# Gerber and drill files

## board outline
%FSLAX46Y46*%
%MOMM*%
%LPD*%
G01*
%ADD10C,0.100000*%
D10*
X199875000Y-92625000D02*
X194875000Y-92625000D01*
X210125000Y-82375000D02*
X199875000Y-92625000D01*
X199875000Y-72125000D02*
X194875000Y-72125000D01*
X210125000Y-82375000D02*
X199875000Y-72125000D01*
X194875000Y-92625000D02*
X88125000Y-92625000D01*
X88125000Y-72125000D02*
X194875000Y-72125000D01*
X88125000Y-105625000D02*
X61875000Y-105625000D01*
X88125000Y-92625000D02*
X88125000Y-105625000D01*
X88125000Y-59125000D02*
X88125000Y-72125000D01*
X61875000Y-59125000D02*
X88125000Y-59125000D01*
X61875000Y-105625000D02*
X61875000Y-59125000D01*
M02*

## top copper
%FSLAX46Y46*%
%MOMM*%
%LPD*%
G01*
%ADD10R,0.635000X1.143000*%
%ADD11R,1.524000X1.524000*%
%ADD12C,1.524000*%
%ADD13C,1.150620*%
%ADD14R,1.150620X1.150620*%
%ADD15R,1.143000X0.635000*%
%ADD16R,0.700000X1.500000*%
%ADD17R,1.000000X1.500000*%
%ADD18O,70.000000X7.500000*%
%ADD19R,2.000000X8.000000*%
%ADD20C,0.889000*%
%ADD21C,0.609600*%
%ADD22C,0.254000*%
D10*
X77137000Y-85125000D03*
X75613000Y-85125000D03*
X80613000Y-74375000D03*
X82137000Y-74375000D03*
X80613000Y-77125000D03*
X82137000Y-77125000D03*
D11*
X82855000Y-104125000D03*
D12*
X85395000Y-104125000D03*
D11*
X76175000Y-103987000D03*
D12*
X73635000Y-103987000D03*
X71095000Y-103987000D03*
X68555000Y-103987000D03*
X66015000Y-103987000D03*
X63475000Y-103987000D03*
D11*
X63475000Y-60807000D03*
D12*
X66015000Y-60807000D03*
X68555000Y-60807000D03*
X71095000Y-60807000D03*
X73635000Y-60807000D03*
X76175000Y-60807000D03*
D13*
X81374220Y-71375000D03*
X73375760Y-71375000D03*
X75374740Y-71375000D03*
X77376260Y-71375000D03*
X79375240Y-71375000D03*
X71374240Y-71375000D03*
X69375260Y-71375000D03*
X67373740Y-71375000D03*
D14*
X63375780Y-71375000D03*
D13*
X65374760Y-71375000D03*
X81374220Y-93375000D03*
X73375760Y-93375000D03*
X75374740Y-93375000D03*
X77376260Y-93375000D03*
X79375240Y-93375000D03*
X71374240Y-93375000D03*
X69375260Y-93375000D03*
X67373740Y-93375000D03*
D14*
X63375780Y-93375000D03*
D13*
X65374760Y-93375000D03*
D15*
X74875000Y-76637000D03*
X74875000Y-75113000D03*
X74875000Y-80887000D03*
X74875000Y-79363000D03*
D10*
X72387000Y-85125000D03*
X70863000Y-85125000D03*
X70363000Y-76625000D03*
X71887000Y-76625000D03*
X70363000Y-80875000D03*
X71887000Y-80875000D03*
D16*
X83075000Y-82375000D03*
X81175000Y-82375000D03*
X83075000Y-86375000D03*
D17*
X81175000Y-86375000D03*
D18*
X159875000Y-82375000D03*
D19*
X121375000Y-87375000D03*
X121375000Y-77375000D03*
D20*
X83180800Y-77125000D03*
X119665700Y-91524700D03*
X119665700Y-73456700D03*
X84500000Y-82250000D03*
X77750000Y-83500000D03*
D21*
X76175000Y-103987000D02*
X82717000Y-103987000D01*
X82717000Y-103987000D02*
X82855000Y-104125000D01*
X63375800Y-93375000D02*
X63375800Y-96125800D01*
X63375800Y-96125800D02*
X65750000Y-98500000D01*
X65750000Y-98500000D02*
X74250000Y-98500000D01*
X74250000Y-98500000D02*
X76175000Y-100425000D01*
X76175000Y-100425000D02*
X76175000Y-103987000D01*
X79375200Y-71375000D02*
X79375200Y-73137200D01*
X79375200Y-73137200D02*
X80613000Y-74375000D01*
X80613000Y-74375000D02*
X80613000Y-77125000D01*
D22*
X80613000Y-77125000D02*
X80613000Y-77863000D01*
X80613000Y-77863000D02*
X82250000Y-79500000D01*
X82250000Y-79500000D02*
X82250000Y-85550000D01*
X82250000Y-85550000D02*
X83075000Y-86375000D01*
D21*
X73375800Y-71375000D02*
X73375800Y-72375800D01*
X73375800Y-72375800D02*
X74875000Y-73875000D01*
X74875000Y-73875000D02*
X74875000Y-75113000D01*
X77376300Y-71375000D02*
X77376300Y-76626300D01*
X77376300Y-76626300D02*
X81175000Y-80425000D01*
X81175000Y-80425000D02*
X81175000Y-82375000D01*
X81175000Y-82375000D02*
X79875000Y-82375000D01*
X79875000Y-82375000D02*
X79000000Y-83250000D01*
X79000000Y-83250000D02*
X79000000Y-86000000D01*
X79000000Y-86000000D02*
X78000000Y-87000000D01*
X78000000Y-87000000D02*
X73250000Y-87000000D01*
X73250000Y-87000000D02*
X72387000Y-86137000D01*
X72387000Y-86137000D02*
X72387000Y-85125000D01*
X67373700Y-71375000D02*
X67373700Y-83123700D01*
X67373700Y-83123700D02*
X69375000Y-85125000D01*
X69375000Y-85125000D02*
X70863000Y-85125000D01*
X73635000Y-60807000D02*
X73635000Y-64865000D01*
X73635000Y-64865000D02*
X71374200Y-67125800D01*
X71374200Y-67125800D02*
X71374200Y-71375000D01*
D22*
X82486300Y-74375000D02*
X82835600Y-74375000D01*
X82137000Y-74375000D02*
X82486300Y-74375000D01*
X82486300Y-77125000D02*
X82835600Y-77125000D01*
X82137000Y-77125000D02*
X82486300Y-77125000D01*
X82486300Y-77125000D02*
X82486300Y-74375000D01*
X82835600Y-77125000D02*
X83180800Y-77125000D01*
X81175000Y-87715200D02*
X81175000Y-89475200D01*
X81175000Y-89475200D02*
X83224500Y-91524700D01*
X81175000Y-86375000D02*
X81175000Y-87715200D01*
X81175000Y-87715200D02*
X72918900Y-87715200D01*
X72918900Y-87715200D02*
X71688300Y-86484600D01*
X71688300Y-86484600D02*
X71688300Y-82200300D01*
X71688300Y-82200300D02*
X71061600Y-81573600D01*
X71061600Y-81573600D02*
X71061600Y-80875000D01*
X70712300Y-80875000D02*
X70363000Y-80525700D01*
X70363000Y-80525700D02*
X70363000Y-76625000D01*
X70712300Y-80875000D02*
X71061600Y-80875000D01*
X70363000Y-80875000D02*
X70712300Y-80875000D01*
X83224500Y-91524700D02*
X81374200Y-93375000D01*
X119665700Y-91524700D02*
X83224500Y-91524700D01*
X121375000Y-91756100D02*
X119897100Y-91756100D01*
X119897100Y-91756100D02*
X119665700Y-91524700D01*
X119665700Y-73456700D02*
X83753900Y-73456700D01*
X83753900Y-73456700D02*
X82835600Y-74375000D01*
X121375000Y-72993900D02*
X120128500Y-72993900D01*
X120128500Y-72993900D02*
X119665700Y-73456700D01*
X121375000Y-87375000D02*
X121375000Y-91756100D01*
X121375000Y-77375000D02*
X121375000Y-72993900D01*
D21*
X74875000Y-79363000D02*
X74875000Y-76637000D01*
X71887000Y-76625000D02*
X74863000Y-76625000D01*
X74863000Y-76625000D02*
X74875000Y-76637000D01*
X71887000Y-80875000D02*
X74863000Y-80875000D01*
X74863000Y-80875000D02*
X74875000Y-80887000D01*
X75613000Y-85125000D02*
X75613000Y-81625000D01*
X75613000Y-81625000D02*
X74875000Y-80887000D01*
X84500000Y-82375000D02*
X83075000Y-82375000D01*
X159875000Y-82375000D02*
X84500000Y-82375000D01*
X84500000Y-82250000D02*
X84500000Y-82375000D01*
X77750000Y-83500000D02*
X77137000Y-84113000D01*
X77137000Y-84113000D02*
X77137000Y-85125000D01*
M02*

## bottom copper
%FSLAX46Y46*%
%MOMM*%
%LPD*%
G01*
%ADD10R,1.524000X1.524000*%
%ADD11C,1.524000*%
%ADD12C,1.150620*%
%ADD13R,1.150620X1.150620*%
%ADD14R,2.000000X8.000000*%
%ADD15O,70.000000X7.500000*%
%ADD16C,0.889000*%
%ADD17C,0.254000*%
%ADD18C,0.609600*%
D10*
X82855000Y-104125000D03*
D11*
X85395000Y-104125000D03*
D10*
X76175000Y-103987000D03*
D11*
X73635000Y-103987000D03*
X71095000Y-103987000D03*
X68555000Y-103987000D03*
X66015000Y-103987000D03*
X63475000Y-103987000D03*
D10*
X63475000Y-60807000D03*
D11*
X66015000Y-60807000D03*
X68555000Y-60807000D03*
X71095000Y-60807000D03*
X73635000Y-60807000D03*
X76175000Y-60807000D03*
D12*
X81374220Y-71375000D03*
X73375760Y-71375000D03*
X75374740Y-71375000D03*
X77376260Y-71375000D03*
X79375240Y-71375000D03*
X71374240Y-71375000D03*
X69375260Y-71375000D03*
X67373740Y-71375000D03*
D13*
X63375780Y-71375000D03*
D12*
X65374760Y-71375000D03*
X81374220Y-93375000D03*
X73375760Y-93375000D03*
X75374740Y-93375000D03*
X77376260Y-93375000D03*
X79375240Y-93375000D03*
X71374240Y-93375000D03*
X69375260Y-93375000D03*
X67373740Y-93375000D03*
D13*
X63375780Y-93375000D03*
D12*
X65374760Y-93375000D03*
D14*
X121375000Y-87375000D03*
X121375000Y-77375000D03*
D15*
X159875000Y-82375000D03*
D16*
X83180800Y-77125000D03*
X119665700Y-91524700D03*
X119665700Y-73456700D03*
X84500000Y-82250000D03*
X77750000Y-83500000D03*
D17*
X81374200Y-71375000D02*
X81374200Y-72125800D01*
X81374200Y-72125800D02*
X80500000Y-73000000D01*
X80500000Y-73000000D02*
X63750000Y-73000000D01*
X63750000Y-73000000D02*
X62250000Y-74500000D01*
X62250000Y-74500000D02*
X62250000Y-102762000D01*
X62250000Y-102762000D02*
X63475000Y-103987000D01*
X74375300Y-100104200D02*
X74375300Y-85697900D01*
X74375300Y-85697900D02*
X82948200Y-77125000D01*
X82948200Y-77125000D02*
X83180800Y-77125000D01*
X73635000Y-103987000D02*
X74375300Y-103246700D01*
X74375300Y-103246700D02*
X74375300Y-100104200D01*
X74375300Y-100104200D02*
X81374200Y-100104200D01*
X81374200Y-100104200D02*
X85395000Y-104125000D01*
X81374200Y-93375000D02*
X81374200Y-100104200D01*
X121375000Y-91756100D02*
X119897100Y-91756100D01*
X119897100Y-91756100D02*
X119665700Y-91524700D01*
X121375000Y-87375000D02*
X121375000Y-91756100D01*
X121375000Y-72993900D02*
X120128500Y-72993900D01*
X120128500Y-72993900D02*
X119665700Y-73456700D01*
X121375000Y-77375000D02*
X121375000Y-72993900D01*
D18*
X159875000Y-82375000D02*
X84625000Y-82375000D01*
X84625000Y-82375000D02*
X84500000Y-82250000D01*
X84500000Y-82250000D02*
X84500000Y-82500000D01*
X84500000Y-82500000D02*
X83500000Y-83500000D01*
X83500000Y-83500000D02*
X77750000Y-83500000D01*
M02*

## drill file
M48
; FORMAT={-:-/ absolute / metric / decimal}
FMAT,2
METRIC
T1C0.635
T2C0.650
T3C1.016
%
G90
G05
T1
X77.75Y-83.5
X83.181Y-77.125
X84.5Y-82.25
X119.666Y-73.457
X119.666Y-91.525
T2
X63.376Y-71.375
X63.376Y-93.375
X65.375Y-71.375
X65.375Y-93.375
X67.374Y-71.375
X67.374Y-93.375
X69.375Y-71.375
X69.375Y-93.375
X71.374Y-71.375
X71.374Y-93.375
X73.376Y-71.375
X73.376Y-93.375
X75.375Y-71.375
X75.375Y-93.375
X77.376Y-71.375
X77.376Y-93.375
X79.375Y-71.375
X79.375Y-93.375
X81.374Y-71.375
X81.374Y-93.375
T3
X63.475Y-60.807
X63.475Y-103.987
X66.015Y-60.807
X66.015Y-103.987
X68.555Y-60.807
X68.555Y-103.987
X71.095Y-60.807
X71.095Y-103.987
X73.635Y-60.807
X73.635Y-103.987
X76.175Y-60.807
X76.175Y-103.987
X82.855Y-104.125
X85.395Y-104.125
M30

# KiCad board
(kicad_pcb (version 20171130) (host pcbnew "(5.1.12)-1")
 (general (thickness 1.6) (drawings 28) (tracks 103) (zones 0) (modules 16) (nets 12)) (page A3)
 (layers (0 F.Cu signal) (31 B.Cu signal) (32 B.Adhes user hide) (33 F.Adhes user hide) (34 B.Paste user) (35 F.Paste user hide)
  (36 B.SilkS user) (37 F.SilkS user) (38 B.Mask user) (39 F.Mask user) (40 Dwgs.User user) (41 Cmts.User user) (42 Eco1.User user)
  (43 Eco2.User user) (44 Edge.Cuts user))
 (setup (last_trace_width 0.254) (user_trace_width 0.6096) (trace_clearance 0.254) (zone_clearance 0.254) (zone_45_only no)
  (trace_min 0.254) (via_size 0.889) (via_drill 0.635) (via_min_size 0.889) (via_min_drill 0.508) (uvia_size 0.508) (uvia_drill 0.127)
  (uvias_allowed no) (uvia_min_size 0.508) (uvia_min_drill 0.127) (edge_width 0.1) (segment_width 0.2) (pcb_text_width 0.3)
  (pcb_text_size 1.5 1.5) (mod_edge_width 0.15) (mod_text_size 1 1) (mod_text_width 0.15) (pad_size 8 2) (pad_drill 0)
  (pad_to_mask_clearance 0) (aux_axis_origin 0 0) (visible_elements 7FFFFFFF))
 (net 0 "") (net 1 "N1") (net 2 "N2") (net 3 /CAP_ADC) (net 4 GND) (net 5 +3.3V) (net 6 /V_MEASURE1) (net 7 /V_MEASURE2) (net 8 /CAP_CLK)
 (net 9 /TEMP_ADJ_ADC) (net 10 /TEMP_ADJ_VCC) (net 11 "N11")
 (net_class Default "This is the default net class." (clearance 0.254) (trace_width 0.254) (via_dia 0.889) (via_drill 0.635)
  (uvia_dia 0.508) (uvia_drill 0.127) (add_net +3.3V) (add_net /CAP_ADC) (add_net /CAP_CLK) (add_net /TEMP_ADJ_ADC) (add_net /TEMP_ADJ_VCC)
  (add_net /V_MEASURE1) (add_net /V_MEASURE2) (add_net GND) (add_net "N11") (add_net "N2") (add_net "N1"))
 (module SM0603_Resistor (layer F.Cu) (at 76.375 85.125 180)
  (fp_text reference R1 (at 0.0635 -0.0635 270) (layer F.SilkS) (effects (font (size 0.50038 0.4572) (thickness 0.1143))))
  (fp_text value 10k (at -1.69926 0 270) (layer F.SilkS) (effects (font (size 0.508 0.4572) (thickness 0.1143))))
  (pad 1 smd rect (at -0.762 0 180) (size 0.635 1.143) (layers F.Cu F.Paste F.Mask) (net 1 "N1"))
  (pad 2 smd rect (at 0.762 0 180) (size 0.635 1.143) (layers F.Cu F.Paste F.Mask) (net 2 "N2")))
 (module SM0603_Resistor (layer F.Cu) (at 81.375 74.375)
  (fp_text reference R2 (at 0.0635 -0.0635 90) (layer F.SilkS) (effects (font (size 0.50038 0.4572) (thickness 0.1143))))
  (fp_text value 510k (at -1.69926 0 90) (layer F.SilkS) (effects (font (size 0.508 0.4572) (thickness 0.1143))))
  (pad 1 smd rect (at -0.762 0) (size 0.635 1.143) (layers F.Cu F.Paste F.Mask) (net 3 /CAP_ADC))
  (pad 2 smd rect (at 0.762 0) (size 0.635 1.143) (layers F.Cu F.Paste F.Mask) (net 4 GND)))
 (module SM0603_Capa (layer F.Cu) (at 81.375 77.125)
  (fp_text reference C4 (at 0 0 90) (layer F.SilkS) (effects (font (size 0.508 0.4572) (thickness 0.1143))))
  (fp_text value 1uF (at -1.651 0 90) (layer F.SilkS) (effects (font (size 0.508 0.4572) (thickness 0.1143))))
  (pad 1 smd rect (at -0.762 0) (size 0.635 1.143) (layers F.Cu F.Paste F.Mask) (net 3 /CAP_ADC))
  (pad 2 smd rect (at 0.762 0) (size 0.635 1.143) (layers F.Cu F.Paste F.Mask) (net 4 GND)))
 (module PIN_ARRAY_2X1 (layer F.Cu) (at 84.125 104.125)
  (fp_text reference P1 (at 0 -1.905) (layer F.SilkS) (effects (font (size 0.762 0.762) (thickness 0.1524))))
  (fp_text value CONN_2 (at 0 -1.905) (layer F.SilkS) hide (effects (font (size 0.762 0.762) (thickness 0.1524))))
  (pad 1 thru_hole rect (at -1.27 0) (size 1.524 1.524) (drill 1.016) (layers *.Cu *.Mask F.SilkS) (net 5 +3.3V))
  (pad 2 thru_hole circle (at 1.27 0) (size 1.524 1.524) (drill 1.016) (layers *.Cu *.Mask F.SilkS) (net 4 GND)))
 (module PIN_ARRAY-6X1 (layer F.Cu) (at 69.825 103.987 180)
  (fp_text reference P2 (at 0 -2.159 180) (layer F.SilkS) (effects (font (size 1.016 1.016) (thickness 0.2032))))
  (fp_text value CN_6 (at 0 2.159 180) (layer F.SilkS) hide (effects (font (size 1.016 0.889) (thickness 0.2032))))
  (pad 1 thru_hole rect (at -6.35 0 180) (size 1.524 1.524) (drill 1.016) (layers *.Cu *.Mask F.SilkS) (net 5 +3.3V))
  (pad 2 thru_hole circle (at -3.81 0 180) (size 1.524 1.524) (drill 1.016) (layers *.Cu *.Mask F.SilkS) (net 4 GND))
  (pad 3 thru_hole circle (at -1.27 0 180) (size 1.524 1.524) (drill 1.016) (layers *.Cu *.Mask F.SilkS))
  (pad 4 thru_hole circle (at 1.27 0 180) (size 1.524 1.524) (drill 1.016) (layers *.Cu *.Mask F.SilkS))
  (pad 5 thru_hole circle (at 3.81 0 180) (size 1.524 1.524) (drill 1.016) (layers *.Cu *.Mask F.SilkS))
  (pad 6 thru_hole circle (at 6.35 0 180) (size 1.524 1.524) (drill 1.016) (layers *.Cu *.Mask F.SilkS) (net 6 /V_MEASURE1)))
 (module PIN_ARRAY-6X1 (layer F.Cu) (at 69.825 60.807)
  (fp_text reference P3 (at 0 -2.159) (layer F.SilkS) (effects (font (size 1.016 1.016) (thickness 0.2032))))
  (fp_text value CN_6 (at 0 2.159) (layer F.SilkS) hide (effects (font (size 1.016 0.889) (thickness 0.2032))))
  (pad 1 thru_hole rect (at -6.35 0) (size 1.524 1.524) (drill 1.016) (layers *.Cu *.Mask F.SilkS))
  (pad 2 thru_hole circle (at -3.81 0) (size 1.524 1.524) (drill 1.016) (layers *.Cu *.Mask F.SilkS))
  (pad 3 thru_hole circle (at -1.27 0) (size 1.524 1.524) (drill 1.016) (layers *.Cu *.Mask F.SilkS))
  (pad 4 thru_hole circle (at 1.27 0) (size 1.524 1.524) (drill 1.016) (layers *.Cu *.Mask F.SilkS))
  (pad 5 thru_hole circle (at 3.81 0) (size 1.524 1.524) (drill 1.016) (layers *.Cu *.Mask F.SilkS) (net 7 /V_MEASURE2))
  (pad 6 thru_hole circle (at 6.35 0) (size 1.524 1.524) (drill 1.016) (layers *.Cu *.Mask F.SilkS)))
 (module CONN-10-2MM (layer F.Cu) (at 72.375 71.375)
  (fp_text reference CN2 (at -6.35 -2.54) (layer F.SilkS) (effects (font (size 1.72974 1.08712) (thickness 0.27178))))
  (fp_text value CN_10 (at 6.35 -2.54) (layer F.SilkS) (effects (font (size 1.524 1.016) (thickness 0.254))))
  (pad 10 thru_hole circle (at 8.99922 0) (size 1.15062 1.15062) (drill 0.65024) (layers *.Cu *.Mask F.SilkS) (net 6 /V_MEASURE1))
  (pad 6 thru_hole circle (at 1.00076 0) (size 1.15062 1.15062) (drill 0.65024) (layers *.Cu *.Mask F.SilkS) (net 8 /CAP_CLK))
  (pad 7 thru_hole circle (at 2.99974 0) (size 1.15062 1.15062) (drill 0.65024) (layers *.Cu *.Mask F.SilkS))
  (pad 8 thru_hole circle (at 5.00126 0) (size 1.15062 1.15062) (drill 0.65024) (layers *.Cu *.Mask F.SilkS) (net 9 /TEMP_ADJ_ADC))
  (pad 9 thru_hole circle (at 7.00024 0) (size 1.15062 1.15062) (drill 0.65024) (layers *.Cu *.Mask F.SilkS) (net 3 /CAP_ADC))
  (pad 5 thru_hole circle (at -1.00076 0) (size 1.15062 1.15062) (drill 0.65024) (layers *.Cu *.Mask F.SilkS) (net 7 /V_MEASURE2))
  (pad 4 thru_hole circle (at -2.99974 0) (size 1.15062 1.15062) (drill 0.65024) (layers *.Cu *.Mask F.SilkS))
  (pad 3 thru_hole circle (at -5.00126 0) (size 1.15062 1.15062) (drill 0.65024) (layers *.Cu *.Mask F.SilkS) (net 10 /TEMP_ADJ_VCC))
  (pad 1 thru_hole rect (at -8.99922 0) (size 1.15062 1.15062) (drill 0.65024) (layers *.Cu *.Mask F.SilkS))
  (pad 2 thru_hole circle (at -7.00024 0) (size 1.15062 1.15062) (drill 0.65024) (layers *.Cu *.Mask F.SilkS)))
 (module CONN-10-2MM (layer F.Cu) (at 72.375 93.375)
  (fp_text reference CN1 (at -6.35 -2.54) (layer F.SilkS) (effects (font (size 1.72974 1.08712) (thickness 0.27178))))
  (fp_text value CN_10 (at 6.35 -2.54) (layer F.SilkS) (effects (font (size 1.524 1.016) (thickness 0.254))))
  (pad 10 thru_hole circle (at 8.99922 0) (size 1.15062 1.15062) (drill 0.65024) (layers *.Cu *.Mask F.SilkS) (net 4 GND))
  (pad 6 thru_hole circle (at 1.00076 0) (size 1.15062 1.15062) (drill 0.65024) (layers *.Cu *.Mask F.SilkS))
  (pad 7 thru_hole circle (at 2.99974 0) (size 1.15062 1.15062) (drill 0.65024) (layers *.Cu *.Mask F.SilkS))
  (pad 8 thru_hole circle (at 5.00126 0) (size 1.15062 1.15062) (drill 0.65024) (layers *.Cu *.Mask F.SilkS))
  (pad 9 thru_hole circle (at 7.00024 0) (size 1.15062 1.15062) (drill 0.65024) (layers *.Cu *.Mask F.SilkS))
  (pad 5 thru_hole circle (at -1.00076 0) (size 1.15062 1.15062) (drill 0.65024) (layers *.Cu *.Mask F.SilkS))
  (pad 4 thru_hole circle (at -2.99974 0) (size 1.15062 1.15062) (drill 0.65024) (layers *.Cu *.Mask F.SilkS))
  (pad 3 thru_hole circle (at -5.00126 0) (size 1.15062 1.15062) (drill 0.65024) (layers *.Cu *.Mask F.SilkS))
  (pad 1 thru_hole rect (at -8.99922 0) (size 1.15062 1.15062) (drill 0.65024) (layers *.Cu *.Mask F.SilkS) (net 5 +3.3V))
  (pad 2 thru_hole circle (at -7.00024 0) (size 1.15062 1.15062) (drill 0.65024) (layers *.Cu *.Mask F.SilkS)))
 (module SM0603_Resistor (layer F.Cu) (at 74.875 75.875 90)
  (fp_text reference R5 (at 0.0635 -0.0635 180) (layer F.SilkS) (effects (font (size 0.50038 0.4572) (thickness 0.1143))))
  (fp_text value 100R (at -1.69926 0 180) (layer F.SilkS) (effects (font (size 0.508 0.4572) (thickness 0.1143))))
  (pad 1 smd rect (at -0.762 0 90) (size 0.635 1.143) (layers F.Cu F.Paste F.Mask) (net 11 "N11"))
  (pad 2 smd rect (at 0.762 0 90) (size 0.635 1.143) (layers F.Cu F.Paste F.Mask) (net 8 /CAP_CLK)))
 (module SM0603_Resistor (layer F.Cu) (at 74.875 80.125 90)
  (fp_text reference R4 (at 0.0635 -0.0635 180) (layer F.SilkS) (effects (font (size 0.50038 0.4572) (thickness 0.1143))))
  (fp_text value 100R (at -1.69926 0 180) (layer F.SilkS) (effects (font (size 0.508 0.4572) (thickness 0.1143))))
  (pad 1 smd rect (at -0.762 0 90) (size 0.635 1.143) (layers F.Cu F.Paste F.Mask) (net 2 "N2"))
  (pad 2 smd rect (at 0.762 0 90) (size 0.635 1.143) (layers F.Cu F.Paste F.Mask) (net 11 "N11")))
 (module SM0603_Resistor (layer F.Cu) (at 71.625 85.125 180)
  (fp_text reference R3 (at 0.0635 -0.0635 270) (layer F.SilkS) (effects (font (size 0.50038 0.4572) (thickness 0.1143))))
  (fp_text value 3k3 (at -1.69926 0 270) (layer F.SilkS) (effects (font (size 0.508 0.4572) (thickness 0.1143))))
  (pad 1 smd rect (at -0.762 0 180) (size 0.635 1.143) (layers F.Cu F.Paste F.Mask) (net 9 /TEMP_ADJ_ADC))
  (pad 2 smd rect (at 0.762 0 180) (size 0.635 1.143) (layers F.Cu F.Paste F.Mask) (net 10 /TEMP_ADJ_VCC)))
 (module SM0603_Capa (layer F.Cu) (at 71.125 76.625)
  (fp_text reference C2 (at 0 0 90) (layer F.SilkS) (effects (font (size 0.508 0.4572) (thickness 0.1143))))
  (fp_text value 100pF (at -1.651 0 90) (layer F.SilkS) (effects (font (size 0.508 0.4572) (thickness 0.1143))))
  (pad 1 smd rect (at -0.762 0) (size 0.635 1.143) (layers F.Cu F.Paste F.Mask) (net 4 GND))
  (pad 2 smd rect (at 0.762 0) (size 0.635 1.143) (layers F.Cu F.Paste F.Mask) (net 11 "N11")))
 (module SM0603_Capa (layer F.Cu) (at 71.125 80.875)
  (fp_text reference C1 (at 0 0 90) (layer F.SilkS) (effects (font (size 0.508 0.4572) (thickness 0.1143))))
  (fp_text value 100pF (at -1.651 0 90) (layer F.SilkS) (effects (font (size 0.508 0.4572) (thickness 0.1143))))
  (pad 1 smd rect (at -0.762 0) (size 0.635 1.143) (layers F.Cu F.Paste F.Mask) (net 4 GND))
  (pad 2 smd rect (at 0.762 0) (size 0.635 1.143) (layers F.Cu F.Paste F.Mask) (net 2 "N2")))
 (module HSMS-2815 (layer F.Cu) (at 82.125 84.375 180)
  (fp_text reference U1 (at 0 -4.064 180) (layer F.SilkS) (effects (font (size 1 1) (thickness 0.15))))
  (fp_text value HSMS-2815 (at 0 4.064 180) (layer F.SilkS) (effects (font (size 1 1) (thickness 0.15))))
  (pad 4 smd rect (at -0.95 2 180) (size 0.7 1.5) (layers F.Cu F.Paste F.Mask) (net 1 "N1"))
  (pad 3 smd rect (at 0.95 2 180) (size 0.7 1.5) (layers F.Cu F.Paste F.Mask) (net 9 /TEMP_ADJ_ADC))
  (pad 2 smd rect (at -0.95 -2 180) (size 0.7 1.5) (layers F.Cu F.Paste F.Mask) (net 3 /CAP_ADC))
  (pad 1 smd rect (at 0.95 -2 180) (size 1 1.5) (layers F.Cu F.Paste F.Mask) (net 4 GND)))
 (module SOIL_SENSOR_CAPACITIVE (layer F.Cu) (at 164.875 82.375 90)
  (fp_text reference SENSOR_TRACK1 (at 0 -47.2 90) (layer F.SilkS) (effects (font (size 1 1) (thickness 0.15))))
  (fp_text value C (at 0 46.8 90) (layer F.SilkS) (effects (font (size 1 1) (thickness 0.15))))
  (pad 1 smd oval (at 0 -5 90) (size 7.5 70) (layers F.Cu) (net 1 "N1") (clearance 2) (zone_connect 2) (thermal_width 0.1) (thermal_gap 2))
  (pad 2 smd rect (at -5 -43.5 90) (size 8 2) (layers F.Cu) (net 4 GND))
  (pad 2 smd rect (at 5 -43.5 90) (size 8 2) (layers F.Cu) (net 4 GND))
  (pad 2 smd rect (at -5 -43.5 90) (size 8 2) (layers B.Cu) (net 4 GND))
  (pad 2 smd rect (at 5 -43.5 90) (size 8 2) (layers B.Cu) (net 4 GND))
  (pad 1 smd oval (at 0 -5 90) (size 7.5 70) (layers B.Cu) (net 1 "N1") (clearance 2) (thermal_width 0.1) (thermal_gap 2)))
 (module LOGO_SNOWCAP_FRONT (layer F.Cu) (at 93.2 82.4 90)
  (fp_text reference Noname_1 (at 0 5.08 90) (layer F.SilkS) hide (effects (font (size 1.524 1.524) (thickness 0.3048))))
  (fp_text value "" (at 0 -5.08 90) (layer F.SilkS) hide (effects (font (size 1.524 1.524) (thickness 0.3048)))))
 (gr_line (start 199.875 92.625) (end 194.875 92.625) (angle 90) (layer Edge.Cuts) (width 0.1))
 (gr_line (start 210.125 82.375) (end 199.875 92.625) (angle 90) (layer Edge.Cuts) (width 0.1))
 (gr_line (start 199.875 72.125) (end 194.875 72.125) (angle 90) (layer Edge.Cuts) (width 0.1))
 (gr_line (start 210.125 82.375) (end 199.875 72.125) (angle 90) (layer Edge.Cuts) (width 0.1))
 (gr_line (start 194.875 92.625) (end 88.125 92.625) (angle 90) (layer Edge.Cuts) (width 0.1))
 (gr_line (start 88.125 72.125) (end 194.875 72.125) (angle 90) (layer Edge.Cuts) (width 0.1))
 (gr_line (start 88.125 105.625) (end 61.875 105.625) (angle 90) (layer Edge.Cuts) (width 0.1))
 (gr_line (start 88.125 92.625) (end 88.125 105.625) (angle 90) (layer Edge.Cuts) (width 0.1))
 (gr_line (start 88.125 59.125) (end 88.125 72.125) (angle 90) (layer Edge.Cuts) (width 0.1))
 (gr_line (start 61.875 59.125) (end 88.125 59.125) (angle 90) (layer Edge.Cuts) (width 0.1))
 (gr_line (start 61.875 105.625) (end 61.875 59.125) (angle 90) (layer Edge.Cuts) (width 0.1))
 (segment (start 76.175 103.987) (end 82.717 103.987) (width 0.6096) (layer F.Cu) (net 5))
 (segment (start 82.717 103.987) (end 82.855 104.125) (width 0.6096) (layer F.Cu) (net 5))
 (segment (start 63.3758 93.375) (end 63.3758 96.1258) (width 0.6096) (layer F.Cu) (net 5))
 (segment (start 63.3758 96.1258) (end 65.75 98.5) (width 0.6096) (layer F.Cu) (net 5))
 (segment (start 65.75 98.5) (end 74.25 98.5) (width 0.6096) (layer F.Cu) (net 5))
 (segment (start 74.25 98.5) (end 76.175 100.425) (width 0.6096) (layer F.Cu) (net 5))
 (segment (start 76.175 100.425) (end 76.175 103.987) (width 0.6096) (layer F.Cu) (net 5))
 (segment (start 79.3752 71.375) (end 79.3752 73.1372) (width 0.6096) (layer F.Cu) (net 3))
 (segment (start 79.3752 73.1372) (end 80.613 74.375) (width 0.6096) (layer F.Cu) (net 3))
 (segment (start 80.613 74.375) (end 80.613 77.125) (width 0.6096) (layer F.Cu) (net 3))
 (segment (start 80.613 77.125) (end 80.613 77.863) (width 0.254) (layer F.Cu) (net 3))
 (segment (start 80.613 77.863) (end 82.25 79.5) (width 0.254) (layer F.Cu) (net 3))
 (segment (start 82.25 79.5) (end 82.25 85.55) (width 0.254) (layer F.Cu) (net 3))
 (segment (start 82.25 85.55) (end 83.075 86.375) (width 0.254) (layer F.Cu) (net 3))
 (segment (start 73.3758 71.375) (end 73.3758 72.3758) (width 0.6096) (layer F.Cu) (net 8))
 (segment (start 73.3758 72.3758) (end 74.875 73.875) (width 0.6096) (layer F.Cu) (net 8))
 (segment (start 74.875 73.875) (end 74.875 75.113) (width 0.6096) (layer F.Cu) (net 8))
 (segment (start 77.3763 71.375) (end 77.3763 76.6263) (width 0.6096) (layer F.Cu) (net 9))
 (segment (start 77.3763 76.6263) (end 81.175 80.425) (width 0.6096) (layer F.Cu) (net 9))
 (segment (start 81.175 80.425) (end 81.175 82.375) (width 0.6096) (layer F.Cu) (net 9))
 (segment (start 81.175 82.375) (end 79.875 82.375) (width 0.6096) (layer F.Cu) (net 9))
 (segment (start 79.875 82.375) (end 79 83.25) (width 0.6096) (layer F.Cu) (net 9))
 (segment (start 79 83.25) (end 79 86) (width 0.6096) (layer F.Cu) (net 9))
 (segment (start 79 86) (end 78 87) (width 0.6096) (layer F.Cu) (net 9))
 (segment (start 78 87) (end 73.25 87) (width 0.6096) (layer F.Cu) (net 9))
 (segment (start 73.25 87) (end 72.387 86.137) (width 0.6096) (layer F.Cu) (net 9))
 (segment (start 72.387 86.137) (end 72.387 85.125) (width 0.6096) (layer F.Cu) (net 9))
 (segment (start 67.3737 71.375) (end 67.3737 83.1237) (width 0.6096) (layer F.Cu) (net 10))
 (segment (start 67.3737 83.1237) (end 69.375 85.125) (width 0.6096) (layer F.Cu) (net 10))
 (segment (start 69.375 85.125) (end 70.863 85.125) (width 0.6096) (layer F.Cu) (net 10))
 (segment (start 81.3742 71.375) (end 81.3742 72.1258) (width 0.254) (layer B.Cu) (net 6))
 (segment (start 81.3742 72.1258) (end 80.5 73) (width 0.254) (layer B.Cu) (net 6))
 (segment (start 80.5 73) (end 63.75 73) (width 0.254) (layer B.Cu) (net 6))
 (segment (start 63.75 73) (end 62.25 74.5) (width 0.254) (layer B.Cu) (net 6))
 (segment (start 62.25 74.5) (end 62.25 102.762) (width 0.254) (layer B.Cu) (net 6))
 (segment (start 62.25 102.762) (end 63.475 103.987) (width 0.254) (layer B.Cu) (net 6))
 (segment (start 73.635 60.807) (end 73.635 64.865) (width 0.6096) (layer F.Cu) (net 7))
 (segment (start 73.635 64.865) (end 71.3742 67.1258) (width 0.6096) (layer F.Cu) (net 7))
 (segment (start 71.3742 67.1258) (end 71.3742 71.375) (width 0.6096) (layer F.Cu) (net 7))
 (segment (start 82.4863 74.375) (end 82.8356 74.375) (width 0.254) (layer F.Cu) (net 4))
 (segment (start 82.137 74.375) (end 82.4863 74.375) (width 0.254) (layer F.Cu) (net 4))
 (segment (start 82.4863 77.125) (end 82.8356 77.125) (width 0.254) (layer F.Cu) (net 4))
 (segment (start 82.137 77.125) (end 82.4863 77.125) (width 0.254) (layer F.Cu) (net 4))
 (segment (start 82.4863 77.125) (end 82.4863 74.375) (width 0.254) (layer F.Cu) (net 4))
 (segment (start 74.3753 100.1042) (end 74.3753 85.6979) (width 0.254) (layer B.Cu) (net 4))
 (segment (start 74.3753 85.6979) (end 82.9482 77.125) (width 0.254) (layer B.Cu) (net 4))
 (segment (start 82.9482 77.125) (end 83.1808 77.125) (width 0.254) (layer B.Cu) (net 4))
 (segment (start 73.635 103.987) (end 74.3753 103.2467) (width 0.254) (layer B.Cu) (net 4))
 (segment (start 74.3753 103.2467) (end 74.3753 100.1042) (width 0.254) (layer B.Cu) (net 4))
 (segment (start 74.3753 100.1042) (end 81.3742 100.1042) (width 0.254) (layer B.Cu) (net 4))
 (segment (start 82.8356 77.125) (end 83.1808 77.125) (width 0.254) (layer F.Cu) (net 4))
 (segment (start 81.175 87.7152) (end 81.175 89.4752) (width 0.254) (layer F.Cu) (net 4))
 (segment (start 81.175 89.4752) (end 83.2245 91.5247) (width 0.254) (layer F.Cu) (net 4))
 (segment (start 81.175 86.375) (end 81.175 87.7152) (width 0.254) (layer F.Cu) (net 4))
 (segment (start 81.175 87.7152) (end 72.9189 87.7152) (width 0.254) (layer F.Cu) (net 4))
 (segment (start 72.9189 87.7152) (end 71.6883 86.4846) (width 0.254) (layer F.Cu) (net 4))
 (segment (start 71.6883 86.4846) (end 71.6883 82.2003) (width 0.254) (layer F.Cu) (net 4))
 (segment (start 71.6883 82.2003) (end 71.0616 81.5736) (width 0.254) (layer F.Cu) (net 4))
 (segment (start 71.0616 81.5736) (end 71.0616 80.875) (width 0.254) (layer F.Cu) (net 4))
 (segment (start 70.7123 80.875) (end 70.363 80.5257) (width 0.254) (layer F.Cu) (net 4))
 (segment (start 70.363 80.5257) (end 70.363 76.625) (width 0.254) (layer F.Cu) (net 4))
 (segment (start 70.7123 80.875) (end 71.0616 80.875) (width 0.254) (layer F.Cu) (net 4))
 (segment (start 70.363 80.875) (end 70.7123 80.875) (width 0.254) (layer F.Cu) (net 4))
 (segment (start 81.3742 100.1042) (end 85.395 104.125) (width 0.254) (layer B.Cu) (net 4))
 (segment (start 81.3742 93.375) (end 81.3742 100.1042) (width 0.254) (layer B.Cu) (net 4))
 (segment (start 83.2245 91.5247) (end 81.3742 93.375) (width 0.254) (layer F.Cu) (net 4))
 (segment (start 119.6657 91.5247) (end 83.2245 91.5247) (width 0.254) (layer F.Cu) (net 4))
 (segment (start 121.375 91.7561) (end 119.8971 91.7561) (width 0.254) (layer B.Cu) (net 4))
 (segment (start 119.8971 91.7561) (end 119.6657 91.5247) (width 0.254) (layer B.Cu) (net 4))
 (segment (start 121.375 91.7561) (end 119.8971 91.7561) (width 0.254) (layer F.Cu) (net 4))
 (segment (start 119.8971 91.7561) (end 119.6657 91.5247) (width 0.254) (layer F.Cu) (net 4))
 (segment (start 119.6657 73.4567) (end 83.7539 73.4567) (width 0.254) (layer F.Cu) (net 4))
 (segment (start 83.7539 73.4567) (end 82.8356 74.375) (width 0.254) (layer F.Cu) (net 4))
 (segment (start 121.375 72.9939) (end 120.1285 72.9939) (width 0.254) (layer F.Cu) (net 4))
 (segment (start 120.1285 72.9939) (end 119.6657 73.4567) (width 0.254) (layer F.Cu) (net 4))
 (segment (start 121.375 87.375) (end 121.375 91.7561) (width 0.254) (layer B.Cu) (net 4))
 (segment (start 121.375 87.375) (end 121.375 91.7561) (width 0.254) (layer F.Cu) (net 4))
 (segment (start 121.375 72.9939) (end 120.1285 72.9939) (width 0.254) (layer B.Cu) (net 4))
 (segment (start 120.1285 72.9939) (end 119.6657 73.4567) (width 0.254) (layer B.Cu) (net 4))
 (segment (start 121.375 77.375) (end 121.375 72.9939) (width 0.254) (layer B.Cu) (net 4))
 (segment (start 121.375 77.375) (end 121.375 72.9939) (width 0.254) (layer F.Cu) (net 4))
 (via (at 83.1808 77.125) (size 0.889) (layers F.Cu B.Cu) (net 4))
 (via (at 119.6657 91.5247) (size 0.889) (layers F.Cu B.Cu) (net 4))
 (via (at 119.6657 73.4567) (size 0.889) (layers F.Cu B.Cu) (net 4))
 (segment (start 74.875 79.363) (end 74.875 76.637) (width 0.6096) (layer F.Cu) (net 11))
 (segment (start 71.887 76.625) (end 74.863 76.625) (width 0.6096) (layer F.Cu) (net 11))
 (segment (start 74.863 76.625) (end 74.875 76.637) (width 0.6096) (layer F.Cu) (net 11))
 (segment (start 71.887 80.875) (end 74.863 80.875) (width 0.6096) (layer F.Cu) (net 2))
 (segment (start 74.863 80.875) (end 74.875 80.887) (width 0.6096) (layer F.Cu) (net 2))
 (segment (start 75.613 85.125) (end 75.613 81.625) (width 0.6096) (layer F.Cu) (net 2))
 (segment (start 75.613 81.625) (end 74.875 80.887) (width 0.6096) (layer F.Cu) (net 2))
 (segment (start 84.5 82.375) (end 83.075 82.375) (width 0.6096) (layer F.Cu) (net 1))
 (segment (start 159.875 82.375) (end 84.5 82.375) (width 0.6096) (layer F.Cu) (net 1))
 (segment (start 159.875 82.375) (end 84.625 82.375) (width 0.6096) (layer B.Cu) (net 1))
 (segment (start 84.625 82.375) (end 84.5 82.25) (width 0.6096) (layer B.Cu) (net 1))
 (segment (start 84.5 82.25) (end 84.5 82.375) (width 0.6096) (layer F.Cu) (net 1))
 (segment (start 84.5 82.25) (end 84.5 82.5) (width 0.6096) (layer B.Cu) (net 1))
 (segment (start 84.5 82.5) (end 83.5 83.5) (width 0.6096) (layer B.Cu) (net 1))
 (segment (start 83.5 83.5) (end 77.75 83.5) (width 0.6096) (layer B.Cu) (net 1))
 (segment (start 77.75 83.5) (end 77.137 84.113) (width 0.6096) (layer F.Cu) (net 1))
 (segment (start 77.137 84.113) (end 77.137 85.125) (width 0.6096) (layer F.Cu) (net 1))
 (via (at 84.5 82.25) (size 0.889) (layers F.Cu B.Cu) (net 1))
 (via (at 77.75 83.5) (size 0.889) (layers F.Cu B.Cu) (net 1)))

